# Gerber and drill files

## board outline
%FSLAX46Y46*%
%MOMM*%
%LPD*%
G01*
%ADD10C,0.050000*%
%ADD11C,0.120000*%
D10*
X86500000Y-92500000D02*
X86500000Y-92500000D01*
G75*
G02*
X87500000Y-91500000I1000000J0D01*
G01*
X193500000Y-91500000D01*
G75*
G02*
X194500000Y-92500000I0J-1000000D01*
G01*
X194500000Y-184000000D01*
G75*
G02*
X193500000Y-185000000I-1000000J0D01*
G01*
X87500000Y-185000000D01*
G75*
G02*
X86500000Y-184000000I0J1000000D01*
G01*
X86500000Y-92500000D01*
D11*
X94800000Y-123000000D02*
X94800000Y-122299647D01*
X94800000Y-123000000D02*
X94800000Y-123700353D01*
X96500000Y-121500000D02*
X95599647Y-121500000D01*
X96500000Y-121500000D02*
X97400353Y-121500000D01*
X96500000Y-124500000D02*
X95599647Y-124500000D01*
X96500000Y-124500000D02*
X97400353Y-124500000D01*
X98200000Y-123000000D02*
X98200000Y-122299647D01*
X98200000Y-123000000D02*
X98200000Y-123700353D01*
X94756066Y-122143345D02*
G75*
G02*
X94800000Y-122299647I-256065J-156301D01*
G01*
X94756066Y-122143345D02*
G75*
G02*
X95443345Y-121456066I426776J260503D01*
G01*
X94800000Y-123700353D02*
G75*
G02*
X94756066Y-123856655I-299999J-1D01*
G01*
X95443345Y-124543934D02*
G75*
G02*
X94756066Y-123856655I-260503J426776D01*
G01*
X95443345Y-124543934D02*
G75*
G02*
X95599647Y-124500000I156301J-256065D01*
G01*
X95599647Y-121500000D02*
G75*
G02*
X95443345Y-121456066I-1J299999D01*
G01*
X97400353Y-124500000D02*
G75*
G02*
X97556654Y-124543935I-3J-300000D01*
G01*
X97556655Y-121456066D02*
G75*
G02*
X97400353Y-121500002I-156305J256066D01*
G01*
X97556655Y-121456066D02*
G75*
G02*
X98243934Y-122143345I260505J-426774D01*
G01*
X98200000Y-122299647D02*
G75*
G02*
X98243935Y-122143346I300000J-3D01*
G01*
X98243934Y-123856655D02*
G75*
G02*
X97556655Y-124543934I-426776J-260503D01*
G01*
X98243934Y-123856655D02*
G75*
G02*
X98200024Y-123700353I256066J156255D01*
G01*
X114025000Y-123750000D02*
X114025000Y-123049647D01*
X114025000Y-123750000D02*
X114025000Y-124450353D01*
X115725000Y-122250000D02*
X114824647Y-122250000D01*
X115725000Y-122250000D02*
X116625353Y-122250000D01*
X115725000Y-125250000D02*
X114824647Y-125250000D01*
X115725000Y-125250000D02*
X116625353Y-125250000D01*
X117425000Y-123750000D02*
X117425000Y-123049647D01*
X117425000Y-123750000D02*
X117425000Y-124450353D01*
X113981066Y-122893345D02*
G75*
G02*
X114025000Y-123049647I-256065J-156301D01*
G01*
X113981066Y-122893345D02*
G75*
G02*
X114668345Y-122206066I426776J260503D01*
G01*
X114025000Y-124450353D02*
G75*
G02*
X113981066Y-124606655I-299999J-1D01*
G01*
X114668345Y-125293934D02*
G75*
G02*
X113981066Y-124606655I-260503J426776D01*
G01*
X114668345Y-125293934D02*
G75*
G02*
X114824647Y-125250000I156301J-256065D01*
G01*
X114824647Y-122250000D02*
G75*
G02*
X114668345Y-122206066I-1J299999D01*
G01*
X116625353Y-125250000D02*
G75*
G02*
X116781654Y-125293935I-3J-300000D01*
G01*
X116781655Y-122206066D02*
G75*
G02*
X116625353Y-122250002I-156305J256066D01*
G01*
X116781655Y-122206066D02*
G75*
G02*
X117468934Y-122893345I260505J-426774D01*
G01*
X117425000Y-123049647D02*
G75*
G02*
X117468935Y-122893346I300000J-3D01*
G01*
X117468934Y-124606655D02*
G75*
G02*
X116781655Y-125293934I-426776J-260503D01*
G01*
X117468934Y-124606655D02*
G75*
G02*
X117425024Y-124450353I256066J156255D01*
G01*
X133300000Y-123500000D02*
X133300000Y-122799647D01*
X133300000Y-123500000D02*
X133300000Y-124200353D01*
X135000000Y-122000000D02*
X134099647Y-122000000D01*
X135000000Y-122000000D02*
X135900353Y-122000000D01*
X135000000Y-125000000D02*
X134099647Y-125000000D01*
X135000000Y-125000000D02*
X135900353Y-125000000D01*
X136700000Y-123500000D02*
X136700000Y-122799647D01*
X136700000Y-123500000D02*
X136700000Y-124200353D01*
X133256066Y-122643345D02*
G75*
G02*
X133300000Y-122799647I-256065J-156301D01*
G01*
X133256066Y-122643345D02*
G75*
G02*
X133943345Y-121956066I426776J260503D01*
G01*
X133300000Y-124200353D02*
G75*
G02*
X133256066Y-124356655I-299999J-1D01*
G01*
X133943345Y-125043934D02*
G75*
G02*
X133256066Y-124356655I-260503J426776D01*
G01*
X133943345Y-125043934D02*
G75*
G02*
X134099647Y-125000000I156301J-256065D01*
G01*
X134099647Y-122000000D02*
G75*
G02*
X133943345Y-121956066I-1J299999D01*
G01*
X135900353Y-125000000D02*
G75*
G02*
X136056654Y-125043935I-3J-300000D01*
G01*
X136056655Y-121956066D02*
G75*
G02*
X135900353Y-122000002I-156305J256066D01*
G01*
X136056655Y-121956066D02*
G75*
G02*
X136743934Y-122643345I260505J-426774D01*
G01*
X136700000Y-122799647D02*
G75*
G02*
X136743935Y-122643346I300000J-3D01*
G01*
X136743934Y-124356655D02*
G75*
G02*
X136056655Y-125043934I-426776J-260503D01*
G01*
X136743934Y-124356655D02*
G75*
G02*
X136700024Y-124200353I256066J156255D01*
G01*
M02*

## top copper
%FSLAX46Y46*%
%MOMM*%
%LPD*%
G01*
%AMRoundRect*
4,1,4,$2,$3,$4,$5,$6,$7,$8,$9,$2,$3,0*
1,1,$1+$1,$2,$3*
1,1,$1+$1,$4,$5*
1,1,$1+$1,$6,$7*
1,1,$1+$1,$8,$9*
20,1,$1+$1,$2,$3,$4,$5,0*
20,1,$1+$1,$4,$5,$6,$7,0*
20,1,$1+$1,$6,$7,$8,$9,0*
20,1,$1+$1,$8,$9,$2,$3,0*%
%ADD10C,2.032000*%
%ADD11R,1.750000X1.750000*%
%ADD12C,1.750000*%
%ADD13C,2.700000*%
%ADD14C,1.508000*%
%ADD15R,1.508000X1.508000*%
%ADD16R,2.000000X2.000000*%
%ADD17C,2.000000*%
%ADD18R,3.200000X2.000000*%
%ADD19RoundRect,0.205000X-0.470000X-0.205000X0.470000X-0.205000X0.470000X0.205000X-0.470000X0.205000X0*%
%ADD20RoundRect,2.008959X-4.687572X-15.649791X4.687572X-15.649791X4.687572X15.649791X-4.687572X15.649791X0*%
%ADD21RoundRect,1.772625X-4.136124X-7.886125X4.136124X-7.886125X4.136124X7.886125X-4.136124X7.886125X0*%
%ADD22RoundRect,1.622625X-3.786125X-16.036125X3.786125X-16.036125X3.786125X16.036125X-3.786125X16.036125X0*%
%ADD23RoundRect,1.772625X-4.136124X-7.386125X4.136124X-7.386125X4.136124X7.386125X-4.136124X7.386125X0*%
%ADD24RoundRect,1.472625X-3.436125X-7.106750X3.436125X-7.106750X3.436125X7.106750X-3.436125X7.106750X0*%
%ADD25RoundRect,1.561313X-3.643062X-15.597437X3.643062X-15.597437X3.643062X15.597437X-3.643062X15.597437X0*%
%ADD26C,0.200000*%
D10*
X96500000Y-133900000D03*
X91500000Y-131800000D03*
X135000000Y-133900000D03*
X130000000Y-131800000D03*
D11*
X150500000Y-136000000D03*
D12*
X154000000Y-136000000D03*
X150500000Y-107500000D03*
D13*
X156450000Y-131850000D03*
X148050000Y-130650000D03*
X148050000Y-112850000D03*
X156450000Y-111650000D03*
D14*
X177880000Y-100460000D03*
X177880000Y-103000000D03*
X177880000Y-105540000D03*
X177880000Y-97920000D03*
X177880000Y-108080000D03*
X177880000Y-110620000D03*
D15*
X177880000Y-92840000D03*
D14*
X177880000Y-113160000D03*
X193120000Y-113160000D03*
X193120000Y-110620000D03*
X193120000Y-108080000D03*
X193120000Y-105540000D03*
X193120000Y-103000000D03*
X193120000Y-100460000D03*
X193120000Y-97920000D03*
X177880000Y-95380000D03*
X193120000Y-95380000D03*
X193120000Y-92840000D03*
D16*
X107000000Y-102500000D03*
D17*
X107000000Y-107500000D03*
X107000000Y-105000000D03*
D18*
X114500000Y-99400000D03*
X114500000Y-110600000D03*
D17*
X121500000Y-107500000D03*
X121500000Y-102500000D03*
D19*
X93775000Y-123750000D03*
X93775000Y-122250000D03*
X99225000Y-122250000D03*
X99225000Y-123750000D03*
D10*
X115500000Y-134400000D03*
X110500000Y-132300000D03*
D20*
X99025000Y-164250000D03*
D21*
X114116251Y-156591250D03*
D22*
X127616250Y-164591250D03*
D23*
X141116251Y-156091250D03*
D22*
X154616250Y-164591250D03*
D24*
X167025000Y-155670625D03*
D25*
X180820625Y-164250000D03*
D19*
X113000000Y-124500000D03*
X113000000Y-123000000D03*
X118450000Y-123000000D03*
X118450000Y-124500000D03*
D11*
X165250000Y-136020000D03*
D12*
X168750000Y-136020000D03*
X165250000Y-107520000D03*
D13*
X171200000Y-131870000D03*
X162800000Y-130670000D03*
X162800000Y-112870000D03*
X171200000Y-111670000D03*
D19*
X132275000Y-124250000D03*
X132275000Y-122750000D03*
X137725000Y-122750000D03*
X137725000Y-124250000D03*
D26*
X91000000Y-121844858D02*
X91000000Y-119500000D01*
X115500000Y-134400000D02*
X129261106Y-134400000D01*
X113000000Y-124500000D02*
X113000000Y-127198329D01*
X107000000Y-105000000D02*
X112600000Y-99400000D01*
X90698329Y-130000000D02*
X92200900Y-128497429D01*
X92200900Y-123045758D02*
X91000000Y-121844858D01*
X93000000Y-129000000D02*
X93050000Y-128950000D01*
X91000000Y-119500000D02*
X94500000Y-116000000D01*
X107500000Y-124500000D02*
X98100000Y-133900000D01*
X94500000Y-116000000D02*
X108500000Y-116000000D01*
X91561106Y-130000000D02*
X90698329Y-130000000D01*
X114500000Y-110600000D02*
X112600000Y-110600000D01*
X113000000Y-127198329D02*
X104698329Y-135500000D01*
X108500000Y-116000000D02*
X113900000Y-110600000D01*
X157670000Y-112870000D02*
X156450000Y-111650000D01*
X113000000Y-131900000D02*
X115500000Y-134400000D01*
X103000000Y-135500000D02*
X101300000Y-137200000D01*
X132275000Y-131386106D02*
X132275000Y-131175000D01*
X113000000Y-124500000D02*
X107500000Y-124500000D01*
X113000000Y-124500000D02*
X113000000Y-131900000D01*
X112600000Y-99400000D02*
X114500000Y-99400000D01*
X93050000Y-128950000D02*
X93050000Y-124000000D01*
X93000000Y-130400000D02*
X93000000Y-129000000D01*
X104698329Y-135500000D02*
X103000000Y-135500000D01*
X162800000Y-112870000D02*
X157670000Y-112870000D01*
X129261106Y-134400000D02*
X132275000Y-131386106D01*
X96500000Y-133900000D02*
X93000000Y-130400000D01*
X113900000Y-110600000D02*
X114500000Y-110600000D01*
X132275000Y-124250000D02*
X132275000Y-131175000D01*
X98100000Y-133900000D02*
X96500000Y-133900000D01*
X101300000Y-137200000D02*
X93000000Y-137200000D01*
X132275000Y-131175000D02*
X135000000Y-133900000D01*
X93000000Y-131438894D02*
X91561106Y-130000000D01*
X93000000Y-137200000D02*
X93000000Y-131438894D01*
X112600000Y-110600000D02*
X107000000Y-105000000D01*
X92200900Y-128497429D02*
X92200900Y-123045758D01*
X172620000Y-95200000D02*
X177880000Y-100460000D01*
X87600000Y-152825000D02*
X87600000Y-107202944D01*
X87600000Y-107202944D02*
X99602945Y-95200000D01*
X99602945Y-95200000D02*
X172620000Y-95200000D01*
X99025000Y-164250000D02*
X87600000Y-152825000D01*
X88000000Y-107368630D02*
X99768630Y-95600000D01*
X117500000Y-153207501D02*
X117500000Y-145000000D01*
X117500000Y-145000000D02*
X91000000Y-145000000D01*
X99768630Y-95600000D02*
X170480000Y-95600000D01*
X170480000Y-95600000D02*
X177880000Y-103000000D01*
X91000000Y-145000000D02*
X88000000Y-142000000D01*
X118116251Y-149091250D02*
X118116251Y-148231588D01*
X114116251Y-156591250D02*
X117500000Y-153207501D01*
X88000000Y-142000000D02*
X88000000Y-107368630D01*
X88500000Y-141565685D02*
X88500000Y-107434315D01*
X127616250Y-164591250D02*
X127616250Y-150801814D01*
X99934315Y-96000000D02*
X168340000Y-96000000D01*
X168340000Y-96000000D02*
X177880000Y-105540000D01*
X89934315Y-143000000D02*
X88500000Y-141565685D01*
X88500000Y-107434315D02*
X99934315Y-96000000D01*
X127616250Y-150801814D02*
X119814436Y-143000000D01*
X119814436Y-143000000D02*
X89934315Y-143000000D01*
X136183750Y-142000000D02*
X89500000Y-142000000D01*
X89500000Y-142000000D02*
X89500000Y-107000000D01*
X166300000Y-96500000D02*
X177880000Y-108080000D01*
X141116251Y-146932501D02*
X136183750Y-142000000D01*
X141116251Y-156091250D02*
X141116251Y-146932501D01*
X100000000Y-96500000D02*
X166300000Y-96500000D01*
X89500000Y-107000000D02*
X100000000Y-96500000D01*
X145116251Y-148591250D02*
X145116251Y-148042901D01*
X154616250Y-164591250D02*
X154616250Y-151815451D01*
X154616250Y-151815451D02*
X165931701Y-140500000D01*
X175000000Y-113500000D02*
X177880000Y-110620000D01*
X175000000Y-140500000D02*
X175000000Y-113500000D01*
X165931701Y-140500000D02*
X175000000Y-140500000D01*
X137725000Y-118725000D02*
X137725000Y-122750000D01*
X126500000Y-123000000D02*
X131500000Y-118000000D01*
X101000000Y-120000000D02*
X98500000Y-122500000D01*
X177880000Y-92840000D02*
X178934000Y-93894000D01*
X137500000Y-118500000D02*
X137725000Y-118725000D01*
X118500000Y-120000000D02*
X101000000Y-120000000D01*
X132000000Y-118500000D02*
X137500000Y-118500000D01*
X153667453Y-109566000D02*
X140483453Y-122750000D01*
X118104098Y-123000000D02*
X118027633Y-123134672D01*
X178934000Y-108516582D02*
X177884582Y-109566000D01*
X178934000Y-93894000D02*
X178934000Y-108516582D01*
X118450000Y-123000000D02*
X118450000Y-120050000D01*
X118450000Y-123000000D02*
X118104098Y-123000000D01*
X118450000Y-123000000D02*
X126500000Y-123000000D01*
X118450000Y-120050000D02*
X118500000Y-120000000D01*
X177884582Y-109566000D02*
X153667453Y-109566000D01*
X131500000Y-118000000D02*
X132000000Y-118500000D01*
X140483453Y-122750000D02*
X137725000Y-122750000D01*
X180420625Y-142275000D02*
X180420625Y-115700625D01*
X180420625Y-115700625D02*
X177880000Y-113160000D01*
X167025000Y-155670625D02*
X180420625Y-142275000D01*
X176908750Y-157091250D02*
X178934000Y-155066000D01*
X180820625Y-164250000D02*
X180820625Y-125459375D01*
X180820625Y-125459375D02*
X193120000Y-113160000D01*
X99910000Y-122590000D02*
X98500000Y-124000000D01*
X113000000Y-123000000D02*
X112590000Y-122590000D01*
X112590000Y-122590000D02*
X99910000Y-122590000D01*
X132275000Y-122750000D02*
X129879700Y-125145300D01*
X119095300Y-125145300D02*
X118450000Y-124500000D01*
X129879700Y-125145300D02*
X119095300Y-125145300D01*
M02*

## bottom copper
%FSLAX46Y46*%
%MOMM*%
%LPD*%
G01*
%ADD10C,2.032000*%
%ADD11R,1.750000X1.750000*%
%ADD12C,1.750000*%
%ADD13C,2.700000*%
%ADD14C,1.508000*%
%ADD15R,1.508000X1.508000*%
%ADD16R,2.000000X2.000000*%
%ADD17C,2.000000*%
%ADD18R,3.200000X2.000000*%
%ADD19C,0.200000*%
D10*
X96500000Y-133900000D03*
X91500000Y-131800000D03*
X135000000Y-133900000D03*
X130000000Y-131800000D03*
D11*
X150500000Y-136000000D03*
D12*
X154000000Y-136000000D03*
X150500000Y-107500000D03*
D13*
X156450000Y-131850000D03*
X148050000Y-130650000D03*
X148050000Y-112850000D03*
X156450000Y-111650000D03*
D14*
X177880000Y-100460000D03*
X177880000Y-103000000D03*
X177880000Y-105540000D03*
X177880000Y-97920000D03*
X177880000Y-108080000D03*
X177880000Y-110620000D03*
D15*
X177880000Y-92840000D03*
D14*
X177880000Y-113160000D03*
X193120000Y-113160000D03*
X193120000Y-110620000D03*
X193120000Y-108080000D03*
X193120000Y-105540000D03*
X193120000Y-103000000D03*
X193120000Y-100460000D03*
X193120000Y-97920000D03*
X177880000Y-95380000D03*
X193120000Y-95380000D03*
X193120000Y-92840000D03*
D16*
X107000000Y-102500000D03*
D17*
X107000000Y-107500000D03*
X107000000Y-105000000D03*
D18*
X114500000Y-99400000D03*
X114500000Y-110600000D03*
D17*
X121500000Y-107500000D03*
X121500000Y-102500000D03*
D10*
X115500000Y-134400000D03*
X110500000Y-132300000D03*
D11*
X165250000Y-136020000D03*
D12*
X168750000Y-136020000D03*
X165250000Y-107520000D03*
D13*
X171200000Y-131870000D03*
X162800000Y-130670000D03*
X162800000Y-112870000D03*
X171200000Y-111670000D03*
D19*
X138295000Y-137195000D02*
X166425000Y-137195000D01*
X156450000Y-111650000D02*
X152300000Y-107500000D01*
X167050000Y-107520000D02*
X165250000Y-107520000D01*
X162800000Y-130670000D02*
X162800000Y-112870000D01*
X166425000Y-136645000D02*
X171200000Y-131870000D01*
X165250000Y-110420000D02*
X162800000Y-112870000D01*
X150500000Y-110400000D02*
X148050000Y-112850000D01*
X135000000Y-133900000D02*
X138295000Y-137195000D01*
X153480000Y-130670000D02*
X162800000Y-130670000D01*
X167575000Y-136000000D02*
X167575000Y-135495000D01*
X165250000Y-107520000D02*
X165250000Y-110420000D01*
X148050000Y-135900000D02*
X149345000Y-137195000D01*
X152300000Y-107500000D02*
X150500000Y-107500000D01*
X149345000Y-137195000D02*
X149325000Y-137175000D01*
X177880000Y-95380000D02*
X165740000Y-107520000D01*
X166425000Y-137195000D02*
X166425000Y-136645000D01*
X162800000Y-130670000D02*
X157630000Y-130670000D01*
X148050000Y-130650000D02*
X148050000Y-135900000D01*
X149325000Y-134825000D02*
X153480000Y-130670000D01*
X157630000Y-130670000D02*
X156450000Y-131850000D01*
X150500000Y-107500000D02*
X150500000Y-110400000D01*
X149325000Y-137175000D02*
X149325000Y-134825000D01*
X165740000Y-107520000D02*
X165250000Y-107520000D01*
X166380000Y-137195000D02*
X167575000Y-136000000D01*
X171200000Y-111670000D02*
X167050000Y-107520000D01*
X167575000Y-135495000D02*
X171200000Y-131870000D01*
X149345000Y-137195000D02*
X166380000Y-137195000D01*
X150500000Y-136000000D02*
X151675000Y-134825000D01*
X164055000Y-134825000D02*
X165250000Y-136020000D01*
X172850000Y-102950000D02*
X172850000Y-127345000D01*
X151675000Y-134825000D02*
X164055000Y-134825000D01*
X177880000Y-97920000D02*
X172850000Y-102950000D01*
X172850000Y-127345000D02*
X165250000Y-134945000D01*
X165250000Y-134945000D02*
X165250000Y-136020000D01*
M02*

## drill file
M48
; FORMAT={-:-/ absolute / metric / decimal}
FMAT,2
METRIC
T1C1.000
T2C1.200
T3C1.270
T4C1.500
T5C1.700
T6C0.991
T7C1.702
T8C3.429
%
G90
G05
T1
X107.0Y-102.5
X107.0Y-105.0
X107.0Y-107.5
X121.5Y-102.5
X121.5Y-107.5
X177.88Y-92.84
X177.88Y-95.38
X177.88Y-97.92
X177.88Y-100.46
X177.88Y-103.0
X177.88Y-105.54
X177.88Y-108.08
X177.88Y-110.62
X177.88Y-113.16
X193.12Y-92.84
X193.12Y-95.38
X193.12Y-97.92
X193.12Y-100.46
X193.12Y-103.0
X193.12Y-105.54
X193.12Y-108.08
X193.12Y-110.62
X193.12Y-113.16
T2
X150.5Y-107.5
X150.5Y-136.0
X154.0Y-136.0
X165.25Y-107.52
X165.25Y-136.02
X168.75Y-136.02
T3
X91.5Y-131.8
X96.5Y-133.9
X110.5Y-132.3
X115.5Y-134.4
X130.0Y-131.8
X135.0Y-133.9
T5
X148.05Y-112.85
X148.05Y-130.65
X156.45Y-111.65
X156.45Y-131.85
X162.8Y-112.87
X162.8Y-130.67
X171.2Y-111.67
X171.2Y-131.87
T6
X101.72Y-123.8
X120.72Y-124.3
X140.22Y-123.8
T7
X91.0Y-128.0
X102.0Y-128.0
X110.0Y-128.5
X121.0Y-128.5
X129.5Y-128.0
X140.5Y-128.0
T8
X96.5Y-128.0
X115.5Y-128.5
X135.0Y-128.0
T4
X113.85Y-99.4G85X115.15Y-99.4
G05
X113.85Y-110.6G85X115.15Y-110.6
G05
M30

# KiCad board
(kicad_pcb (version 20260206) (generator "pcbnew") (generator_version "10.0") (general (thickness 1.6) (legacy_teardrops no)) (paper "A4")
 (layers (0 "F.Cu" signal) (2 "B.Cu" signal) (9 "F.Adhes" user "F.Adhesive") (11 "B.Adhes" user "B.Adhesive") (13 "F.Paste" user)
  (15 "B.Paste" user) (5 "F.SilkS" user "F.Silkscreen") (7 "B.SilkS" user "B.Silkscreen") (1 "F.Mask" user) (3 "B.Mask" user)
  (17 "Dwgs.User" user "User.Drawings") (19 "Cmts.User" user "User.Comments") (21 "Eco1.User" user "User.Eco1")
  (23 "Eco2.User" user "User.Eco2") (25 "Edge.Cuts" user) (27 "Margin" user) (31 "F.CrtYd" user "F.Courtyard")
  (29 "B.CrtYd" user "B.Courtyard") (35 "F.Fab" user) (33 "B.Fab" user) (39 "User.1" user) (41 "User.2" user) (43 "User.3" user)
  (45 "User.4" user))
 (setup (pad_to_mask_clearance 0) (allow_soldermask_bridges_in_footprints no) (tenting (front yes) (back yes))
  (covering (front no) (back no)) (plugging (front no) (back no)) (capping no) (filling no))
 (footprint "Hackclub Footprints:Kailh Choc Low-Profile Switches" (layer "F.Cu") (at 96.5 128)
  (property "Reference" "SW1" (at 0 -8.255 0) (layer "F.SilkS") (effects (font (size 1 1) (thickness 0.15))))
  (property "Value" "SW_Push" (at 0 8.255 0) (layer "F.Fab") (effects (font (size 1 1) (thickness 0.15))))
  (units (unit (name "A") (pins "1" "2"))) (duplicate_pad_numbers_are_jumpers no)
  (pad "" np_thru_hole circle (at -5.5 0) (size 1.7018 1.7018) (drill 1.7018) (layers "*.Cu" "*.Mask"))
  (pad "" np_thru_hole circle (at 0 0) (size 3.429 3.429) (drill 3.429) (layers "*.Cu" "*.Mask"))
  (pad "" np_thru_hole circle (at 5.22 -4.2) (size 0.9906 0.9906) (drill 0.9906) (layers "*.Cu" "*.Mask"))
  (pad "" np_thru_hole circle (at 5.5 0) (size 1.7018 1.7018) (drill 1.7018) (layers "*.Cu" "*.Mask"))
  (pad "1" thru_hole circle (at 0 5.9) (size 2.032 2.032) (drill 1.27) (layers "*.Cu" "*.Mask") (remove_unused_layers no) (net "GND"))
  (pad "2" thru_hole circle (at -5 3.8) (size 2.032 2.032) (drill 1.27) (layers "*.Cu" "*.Mask") (remove_unused_layers no) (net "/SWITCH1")))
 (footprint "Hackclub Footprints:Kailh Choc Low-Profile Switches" (layer "F.Cu") (at 135 128)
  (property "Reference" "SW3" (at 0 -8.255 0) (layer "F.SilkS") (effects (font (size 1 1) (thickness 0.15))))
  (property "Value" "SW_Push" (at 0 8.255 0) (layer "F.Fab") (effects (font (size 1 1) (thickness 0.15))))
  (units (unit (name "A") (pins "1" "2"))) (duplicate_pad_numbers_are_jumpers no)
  (pad "" np_thru_hole circle (at -5.5 0) (size 1.7018 1.7018) (drill 1.7018) (layers "*.Cu" "*.Mask"))
  (pad "" np_thru_hole circle (at 0 0) (size 3.429 3.429) (drill 3.429) (layers "*.Cu" "*.Mask"))
  (pad "" np_thru_hole circle (at 5.22 -4.2) (size 0.9906 0.9906) (drill 0.9906) (layers "*.Cu" "*.Mask"))
  (pad "" np_thru_hole circle (at 5.5 0) (size 1.7018 1.7018) (drill 1.7018) (layers "*.Cu" "*.Mask"))
  (pad "1" thru_hole circle (at 0 5.9) (size 2.032 2.032) (drill 1.27) (layers "*.Cu" "*.Mask") (remove_unused_layers no) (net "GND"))
  (pad "2" thru_hole circle (at -5 3.8) (size 2.032 2.032) (drill 1.27) (layers "*.Cu" "*.Mask") (remove_unused_layers no) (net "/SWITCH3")))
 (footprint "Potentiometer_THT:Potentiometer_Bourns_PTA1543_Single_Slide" (layer "F.Cu") (at 150.5 136 90)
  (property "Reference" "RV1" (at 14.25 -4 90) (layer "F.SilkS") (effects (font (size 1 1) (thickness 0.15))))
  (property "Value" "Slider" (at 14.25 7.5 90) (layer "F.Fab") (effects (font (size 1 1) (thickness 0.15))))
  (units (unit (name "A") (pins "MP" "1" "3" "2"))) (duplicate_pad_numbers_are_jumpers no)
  (pad "1" thru_hole rect (at 0 0 90) (size 1.75 1.75) (drill 1.2) (layers "*.Cu" "*.Mask") (remove_unused_layers no) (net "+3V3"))
  (pad "2" thru_hole circle (at 0 3.5 90) (size 1.75 1.75) (drill 1.2) (layers "*.Cu" "*.Mask") (remove_unused_layers no) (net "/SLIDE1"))
  (pad "3" thru_hole circle (at 28.5 0 90) (size 1.75 1.75) (drill 1.2) (layers "*.Cu" "*.Mask") (remove_unused_layers no) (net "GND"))
  (pad "MP" thru_hole circle (at 4.15 5.95 90) (size 2.7 2.7) (drill 1.7) (layers "*.Cu" "*.Mask") (remove_unused_layers no) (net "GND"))
  (pad "MP" thru_hole circle (at 5.35 -2.45 90) (size 2.7 2.7) (drill 1.7) (layers "*.Cu" "*.Mask") (remove_unused_layers no) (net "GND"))
  (pad "MP" thru_hole circle (at 23.15 -2.45 90) (size 2.7 2.7) (drill 1.7) (layers "*.Cu" "*.Mask") (remove_unused_layers no) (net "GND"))
  (pad "MP" thru_hole circle (at 24.35 5.95 90) (size 2.7 2.7) (drill 1.7) (layers "*.Cu" "*.Mask") (remove_unused_layers no) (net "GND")))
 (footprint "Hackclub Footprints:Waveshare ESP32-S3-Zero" (layer "F.Cu") (at 185.5 103)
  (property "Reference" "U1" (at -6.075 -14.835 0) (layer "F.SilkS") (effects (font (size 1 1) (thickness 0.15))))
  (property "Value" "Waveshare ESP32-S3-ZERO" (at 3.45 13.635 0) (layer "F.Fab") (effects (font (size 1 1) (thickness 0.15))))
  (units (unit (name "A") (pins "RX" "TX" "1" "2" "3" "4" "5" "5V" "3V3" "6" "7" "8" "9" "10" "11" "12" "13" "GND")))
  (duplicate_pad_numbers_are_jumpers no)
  (pad "1" thru_hole circle (at -7.62 -2.54) (size 1.508 1.508) (drill 1) (layers "*.Cu" "*.Mask") (remove_unused_layers no) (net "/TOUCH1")
   (solder_mask_margin 0.102))
  (pad "2" thru_hole circle (at -7.62 0) (size 1.508 1.508) (drill 1) (layers "*.Cu" "*.Mask") (remove_unused_layers no) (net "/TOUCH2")
   (solder_mask_margin 0.102))
  (pad "3" thru_hole circle (at -7.62 2.54) (size 1.508 1.508) (drill 1) (layers "*.Cu" "*.Mask") (remove_unused_layers no) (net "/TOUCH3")
   (solder_mask_margin 0.102))
  (pad "3V3" thru_hole circle (at -7.62 -5.08) (size 1.508 1.508) (drill 1) (layers "*.Cu" "*.Mask") (remove_unused_layers no) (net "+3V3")
   (solder_mask_margin 0.102))
  (pad "4" thru_hole circle (at -7.62 5.08) (size 1.508 1.508) (drill 1) (layers "*.Cu" "*.Mask") (remove_unused_layers no) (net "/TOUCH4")
   (solder_mask_margin 0.102))
  (pad "5" thru_hole circle (at -7.62 7.62) (size 1.508 1.508) (drill 1) (layers "*.Cu" "*.Mask") (remove_unused_layers no) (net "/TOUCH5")
   (solder_mask_margin 0.102))
  (pad "5V" thru_hole rect (at -7.62 -10.16) (size 1.508 1.508) (drill 1) (layers "*.Cu" "*.Mask") (remove_unused_layers no) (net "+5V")
   (solder_mask_margin 0.102))
  (pad "6" thru_hole circle (at -7.62 10.16) (size 1.508 1.508) (drill 1) (layers "*.Cu" "*.Mask") (remove_unused_layers no) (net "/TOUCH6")
   (solder_mask_margin 0.102))
  (pad "7" thru_hole circle (at 7.62 10.16) (size 1.508 1.508) (drill 1) (layers "*.Cu" "*.Mask") (remove_unused_layers no) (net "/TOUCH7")
   (solder_mask_margin 0.102))
  (pad "8" thru_hole circle (at 7.62 7.62) (size 1.508 1.508) (drill 1) (layers "*.Cu" "*.Mask") (remove_unused_layers no)
   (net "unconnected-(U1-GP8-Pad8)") (solder_mask_margin 0.102))
  (pad "9" thru_hole circle (at 7.62 5.08) (size 1.508 1.508) (drill 1) (layers "*.Cu" "*.Mask") (remove_unused_layers no)
   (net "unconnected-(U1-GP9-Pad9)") (solder_mask_margin 0.102))
  (pad "10" thru_hole circle (at 7.62 2.54) (size 1.508 1.508) (drill 1) (layers "*.Cu" "*.Mask") (remove_unused_layers no)
   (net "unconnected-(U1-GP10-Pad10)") (solder_mask_margin 0.102))
  (pad "11" thru_hole circle (at 7.62 0) (size 1.508 1.508) (drill 1) (layers "*.Cu" "*.Mask") (remove_unused_layers no)
   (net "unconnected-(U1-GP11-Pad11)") (solder_mask_margin 0.102))
  (pad "12" thru_hole circle (at 7.62 -2.54) (size 1.508 1.508) (drill 1) (layers "*.Cu" "*.Mask") (remove_unused_layers no)
   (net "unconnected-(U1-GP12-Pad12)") (solder_mask_margin 0.102))
  (pad "13" thru_hole circle (at 7.62 -5.08) (size 1.508 1.508) (drill 1) (layers "*.Cu" "*.Mask") (remove_unused_layers no)
   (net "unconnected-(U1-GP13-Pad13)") (solder_mask_margin 0.102))
  (pad "GND" thru_hole circle (at -7.62 -7.62) (size 1.508 1.508) (drill 1) (layers "*.Cu" "*.Mask") (remove_unused_layers no) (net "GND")
   (solder_mask_margin 0.102))
  (pad "RX" thru_hole circle (at 7.62 -7.62) (size 1.508 1.508) (drill 1) (layers "*.Cu" "*.Mask") (remove_unused_layers no)
   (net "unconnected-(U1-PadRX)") (solder_mask_margin 0.102))
  (pad "TX" thru_hole circle (at 7.62 -10.16) (size 1.508 1.508) (drill 1) (layers "*.Cu" "*.Mask") (remove_unused_layers no)
   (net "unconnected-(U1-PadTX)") (solder_mask_margin 0.102)))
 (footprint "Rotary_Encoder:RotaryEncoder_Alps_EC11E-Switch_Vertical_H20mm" (layer "F.Cu") (at 107 102.5)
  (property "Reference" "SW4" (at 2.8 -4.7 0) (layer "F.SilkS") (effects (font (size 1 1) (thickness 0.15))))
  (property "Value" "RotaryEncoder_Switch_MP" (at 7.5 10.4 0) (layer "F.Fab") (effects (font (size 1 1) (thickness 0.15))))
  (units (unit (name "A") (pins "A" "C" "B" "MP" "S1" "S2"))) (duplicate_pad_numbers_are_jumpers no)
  (pad "A" thru_hole rect (at 0 0) (size 2 2) (drill 1) (layers "*.Cu" "*.Mask") (remove_unused_layers no) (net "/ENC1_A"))
  (pad "B" thru_hole circle (at 0 5) (size 2 2) (drill 1) (layers "*.Cu" "*.Mask") (remove_unused_layers no) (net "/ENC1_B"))
  (pad "C" thru_hole circle (at 0 2.5) (size 2 2) (drill 1) (layers "*.Cu" "*.Mask") (remove_unused_layers no) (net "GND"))
  (pad "MP" thru_hole rect (at 7.5 -3.1) (size 3.2 2) (drill oval 2.8 1.5) (layers "*.Cu" "*.Mask") (remove_unused_layers no) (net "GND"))
  (pad "MP" thru_hole rect (at 7.5 8.1) (size 3.2 2) (drill oval 2.8 1.5) (layers "*.Cu" "*.Mask") (remove_unused_layers no) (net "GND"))
  (pad "S1" thru_hole circle (at 14.5 5) (size 2 2) (drill 1) (layers "*.Cu" "*.Mask") (remove_unused_layers no)
   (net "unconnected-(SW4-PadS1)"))
  (pad "S2" thru_hole circle (at 14.5 0) (size 2 2) (drill 1) (layers "*.Cu" "*.Mask") (remove_unused_layers no)
   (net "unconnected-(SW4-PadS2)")))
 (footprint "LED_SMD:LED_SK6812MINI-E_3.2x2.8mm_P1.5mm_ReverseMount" (layer "F.Cu") (at 96.5 123)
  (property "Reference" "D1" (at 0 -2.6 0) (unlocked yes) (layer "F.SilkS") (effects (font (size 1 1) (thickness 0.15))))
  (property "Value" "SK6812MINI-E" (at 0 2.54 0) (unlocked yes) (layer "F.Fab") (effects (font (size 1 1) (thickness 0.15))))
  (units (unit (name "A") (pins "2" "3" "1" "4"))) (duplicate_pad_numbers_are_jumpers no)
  (fp_line (start -1.7 0) (end -1.7 -0.700353) (stroke (width 0.12) (type solid)) (layer "Edge.Cuts"))
  (fp_line (start -1.7 0) (end -1.7 0.700353) (stroke (width 0.12) (type solid)) (layer "Edge.Cuts"))
  (fp_line (start 0 -1.5) (end -0.900353 -1.5) (stroke (width 0.12) (type solid)) (layer "Edge.Cuts"))
  (fp_line (start 0 -1.5) (end 0.900353 -1.5) (stroke (width 0.12) (type solid)) (layer "Edge.Cuts"))
  (fp_line (start 0 1.5) (end -0.900353 1.5) (stroke (width 0.12) (type solid)) (layer "Edge.Cuts"))
  (fp_line (start 0 1.5) (end 0.900353 1.5) (stroke (width 0.12) (type solid)) (layer "Edge.Cuts"))
  (fp_line (start 1.7 0) (end 1.7 -0.700353) (stroke (width 0.12) (type solid)) (layer "Edge.Cuts"))
  (fp_line (start 1.7 0) (end 1.7 0.700353) (stroke (width 0.12) (type solid)) (layer "Edge.Cuts"))
  (fp_arc (start -1.743934 -0.856655) (mid -1.711192 -0.781532) (end -1.7 -0.700353) (stroke (width 0.12) (type solid)) (layer "Edge.Cuts"))
  (fp_arc (start -1.743934 -0.856655) (mid -1.670711 -1.470711) (end -1.056655 -1.543934) (stroke (width 0.12) (type solid))
   (layer "Edge.Cuts"))
  (fp_arc (start -1.7 0.700353) (mid -1.711192 0.781532) (end -1.743934 0.856655) (stroke (width 0.12) (type solid)) (layer "Edge.Cuts"))
  (fp_arc (start -1.056655 1.543934) (mid -1.670711 1.470711) (end -1.743934 0.856655) (stroke (width 0.12) (type solid))
   (layer "Edge.Cuts"))
  (fp_arc (start -1.056655 1.543934) (mid -0.981532 1.511192) (end -0.900353 1.5) (stroke (width 0.12) (type solid)) (layer "Edge.Cuts"))
  (fp_arc (start -0.900353 -1.5) (mid -0.981532 -1.511192) (end -1.056655 -1.543934) (stroke (width 0.12) (type solid)) (layer "Edge.Cuts"))
  (fp_arc (start 0.900353 1.5) (mid 0.981532 1.511192) (end 1.056655 1.543934) (stroke (width 0.12) (type solid)) (layer "Edge.Cuts"))
  (fp_arc (start 1.056655 -1.543934) (mid 0.981532 -1.511192) (end 0.900353 -1.5) (stroke (width 0.12) (type solid)) (layer "Edge.Cuts"))
  (fp_arc (start 1.056655 -1.543934) (mid 1.670711 -1.470711) (end 1.743934 -0.856655) (stroke (width 0.12) (type solid))
   (layer "Edge.Cuts"))
  (fp_arc (start 1.7 -0.700353) (mid 1.711192 -0.781532) (end 1.743934 -0.856655) (stroke (width 0.12) (type solid)) (layer "Edge.Cuts"))
  (fp_arc (start 1.743934 0.856655) (mid 1.670711 1.470711) (end 1.056655 1.543934) (stroke (width 0.12) (type solid)) (layer "Edge.Cuts"))
  (fp_arc (start 1.743934 0.856655) (mid 1.711192 0.781532) (end 1.7 0.700353) (stroke (width 0.12) (type solid)) (layer "Edge.Cuts"))
  (pad "1" smd roundrect (at -2.725 0.75) (size 1.35 0.82) (layers "F.Cu" "F.Mask" "F.Paste") (roundrect_rratio 0.25) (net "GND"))
  (pad "2" smd roundrect (at -2.725 -0.75) (size 1.35 0.82) (layers "F.Cu" "F.Mask" "F.Paste") (roundrect_rratio 0.25) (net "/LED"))
  (pad "3" smd roundrect (at 2.725 -0.75) (size 1.35 0.82) (layers "F.Cu" "F.Mask" "F.Paste") (roundrect_rratio 0.25) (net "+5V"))
  (pad "4" smd roundrect (at 2.725 0.75) (size 1.35 0.82) (layers "F.Cu" "F.Mask" "F.Paste") (roundrect_rratio 0.25) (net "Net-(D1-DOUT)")))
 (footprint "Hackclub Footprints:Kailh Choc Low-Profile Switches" (layer "F.Cu") (at 115.5 128.5)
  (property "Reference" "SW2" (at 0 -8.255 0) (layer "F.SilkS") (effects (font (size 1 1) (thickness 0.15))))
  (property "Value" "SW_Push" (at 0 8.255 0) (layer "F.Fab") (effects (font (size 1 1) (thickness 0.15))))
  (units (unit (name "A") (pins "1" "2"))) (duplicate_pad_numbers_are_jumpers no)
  (pad "" np_thru_hole circle (at -5.5 0) (size 1.7018 1.7018) (drill 1.7018) (layers "*.Cu" "*.Mask"))
  (pad "" np_thru_hole circle (at 0 0) (size 3.429 3.429) (drill 3.429) (layers "*.Cu" "*.Mask"))
  (pad "" np_thru_hole circle (at 5.22 -4.2) (size 0.9906 0.9906) (drill 0.9906) (layers "*.Cu" "*.Mask"))
  (pad "" np_thru_hole circle (at 5.5 0) (size 1.7018 1.7018) (drill 1.7018) (layers "*.Cu" "*.Mask"))
  (pad "1" thru_hole circle (at 0 5.9) (size 2.032 2.032) (drill 1.27) (layers "*.Cu" "*.Mask") (remove_unused_layers no) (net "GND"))
  (pad "2" thru_hole circle (at -5 3.8) (size 2.032 2.032) (drill 1.27) (layers "*.Cu" "*.Mask") (remove_unused_layers no) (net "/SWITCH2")))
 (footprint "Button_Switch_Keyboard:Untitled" (layer "F.Cu") (at 141.025 142.25)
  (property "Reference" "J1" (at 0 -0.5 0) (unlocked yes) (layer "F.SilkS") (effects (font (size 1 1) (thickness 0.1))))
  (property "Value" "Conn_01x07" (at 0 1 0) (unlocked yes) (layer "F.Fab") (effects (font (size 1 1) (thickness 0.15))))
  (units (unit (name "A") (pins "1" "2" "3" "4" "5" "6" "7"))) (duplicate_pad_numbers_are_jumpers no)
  (pad "1" smd roundrect (at -42 22) (size 13.393062 35.3175) (layers "F.Cu" "F.Mask") (roundrect_rratio 0.15) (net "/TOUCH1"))
  (pad "2" smd roundrect (at -26.908749 14.34125) (size 11.817498 19.3175) (layers "F.Cu" "F.Mask") (roundrect_rratio 0.15) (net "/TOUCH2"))
  (pad "3" smd roundrect (at -13.40875 22.34125) (size 10.8175 35.3175) (layers "F.Cu" "F.Mask") (roundrect_rratio 0.15) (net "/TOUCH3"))
  (pad "4" smd roundrect (at 0.091251 13.84125) (size 11.817498 18.3175) (layers "F.Cu" "F.Mask") (roundrect_rratio 0.15) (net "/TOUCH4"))
  (pad "5" smd roundrect (at 13.59125 22.34125) (size 10.8175 35.3175) (layers "F.Cu" "F.Mask") (roundrect_rratio 0.15) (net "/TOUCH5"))
  (pad "6" smd roundrect (at 26 13.420625) (size 9.8175 17.15875) (layers "F.Cu" "F.Mask") (roundrect_rratio 0.15) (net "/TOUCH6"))
  (pad "7" smd roundrect (at 39.795625 22) (size 10.40875 34.3175) (layers "F.Cu" "F.Mask") (roundrect_rratio 0.15) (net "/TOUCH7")))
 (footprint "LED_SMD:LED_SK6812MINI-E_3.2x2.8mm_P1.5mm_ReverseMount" (layer "F.Cu") (at 115.725 123.75)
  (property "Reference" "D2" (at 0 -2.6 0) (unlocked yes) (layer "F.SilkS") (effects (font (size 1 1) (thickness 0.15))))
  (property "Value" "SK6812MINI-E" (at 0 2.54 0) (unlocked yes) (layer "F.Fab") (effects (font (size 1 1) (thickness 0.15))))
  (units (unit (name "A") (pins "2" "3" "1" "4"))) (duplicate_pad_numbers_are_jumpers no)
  (fp_line (start -1.7 0) (end -1.7 -0.700353) (stroke (width 0.12) (type solid)) (layer "Edge.Cuts"))
  (fp_line (start -1.7 0) (end -1.7 0.700353) (stroke (width 0.12) (type solid)) (layer "Edge.Cuts"))
  (fp_line (start 0 -1.5) (end -0.900353 -1.5) (stroke (width 0.12) (type solid)) (layer "Edge.Cuts"))
  (fp_line (start 0 -1.5) (end 0.900353 -1.5) (stroke (width 0.12) (type solid)) (layer "Edge.Cuts"))
  (fp_line (start 0 1.5) (end -0.900353 1.5) (stroke (width 0.12) (type solid)) (layer "Edge.Cuts"))
  (fp_line (start 0 1.5) (end 0.900353 1.5) (stroke (width 0.12) (type solid)) (layer "Edge.Cuts"))
  (fp_line (start 1.7 0) (end 1.7 -0.700353) (stroke (width 0.12) (type solid)) (layer "Edge.Cuts"))
  (fp_line (start 1.7 0) (end 1.7 0.700353) (stroke (width 0.12) (type solid)) (layer "Edge.Cuts"))
  (fp_arc (start -1.743934 -0.856655) (mid -1.711192 -0.781532) (end -1.7 -0.700353) (stroke (width 0.12) (type solid)) (layer "Edge.Cuts"))
  (fp_arc (start -1.743934 -0.856655) (mid -1.670711 -1.470711) (end -1.056655 -1.543934) (stroke (width 0.12) (type solid))
   (layer "Edge.Cuts"))
  (fp_arc (start -1.7 0.700353) (mid -1.711192 0.781532) (end -1.743934 0.856655) (stroke (width 0.12) (type solid)) (layer "Edge.Cuts"))
  (fp_arc (start -1.056655 1.543934) (mid -1.670711 1.470711) (end -1.743934 0.856655) (stroke (width 0.12) (type solid))
   (layer "Edge.Cuts"))
  (fp_arc (start -1.056655 1.543934) (mid -0.981532 1.511192) (end -0.900353 1.5) (stroke (width 0.12) (type solid)) (layer "Edge.Cuts"))
  (fp_arc (start -0.900353 -1.5) (mid -0.981532 -1.511192) (end -1.056655 -1.543934) (stroke (width 0.12) (type solid)) (layer "Edge.Cuts"))
  (fp_arc (start 0.900353 1.5) (mid 0.981532 1.511192) (end 1.056655 1.543934) (stroke (width 0.12) (type solid)) (layer "Edge.Cuts"))
  (fp_arc (start 1.056655 -1.543934) (mid 0.981532 -1.511192) (end 0.900353 -1.5) (stroke (width 0.12) (type solid)) (layer "Edge.Cuts"))
  (fp_arc (start 1.056655 -1.543934) (mid 1.670711 -1.470711) (end 1.743934 -0.856655) (stroke (width 0.12) (type solid))
   (layer "Edge.Cuts"))
  (fp_arc (start 1.7 -0.700353) (mid 1.711192 -0.781532) (end 1.743934 -0.856655) (stroke (width 0.12) (type solid)) (layer "Edge.Cuts"))
  (fp_arc (start 1.743934 0.856655) (mid 1.670711 1.470711) (end 1.056655 1.543934) (stroke (width 0.12) (type solid)) (layer "Edge.Cuts"))
  (fp_arc (start 1.743934 0.856655) (mid 1.711192 0.781532) (end 1.7 0.700353) (stroke (width 0.12) (type solid)) (layer "Edge.Cuts"))
  (pad "1" smd roundrect (at -2.725 0.75) (size 1.35 0.82) (layers "F.Cu" "F.Mask" "F.Paste") (roundrect_rratio 0.25) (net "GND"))
  (pad "2" smd roundrect (at -2.725 -0.75) (size 1.35 0.82) (layers "F.Cu" "F.Mask" "F.Paste") (roundrect_rratio 0.25) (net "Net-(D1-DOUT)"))
  (pad "3" smd roundrect (at 2.725 -0.75) (size 1.35 0.82) (layers "F.Cu" "F.Mask" "F.Paste") (roundrect_rratio 0.25) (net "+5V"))
  (pad "4" smd roundrect (at 2.725 0.75) (size 1.35 0.82) (layers "F.Cu" "F.Mask" "F.Paste") (roundrect_rratio 0.25) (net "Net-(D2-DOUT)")))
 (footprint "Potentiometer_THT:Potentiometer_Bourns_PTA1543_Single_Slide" (layer "F.Cu") (at 165.25 136.02 90)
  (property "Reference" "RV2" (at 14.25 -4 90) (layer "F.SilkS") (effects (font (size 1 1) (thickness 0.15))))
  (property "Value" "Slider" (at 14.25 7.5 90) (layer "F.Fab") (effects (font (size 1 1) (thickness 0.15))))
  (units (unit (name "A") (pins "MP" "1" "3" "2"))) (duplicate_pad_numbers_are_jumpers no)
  (pad "1" thru_hole rect (at 0 0 90) (size 1.75 1.75) (drill 1.2) (layers "*.Cu" "*.Mask") (remove_unused_layers no) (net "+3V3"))
  (pad "2" thru_hole circle (at 0 3.5 90) (size 1.75 1.75) (drill 1.2) (layers "*.Cu" "*.Mask") (remove_unused_layers no) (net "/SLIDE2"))
  (pad "3" thru_hole circle (at 28.5 0 90) (size 1.75 1.75) (drill 1.2) (layers "*.Cu" "*.Mask") (remove_unused_layers no) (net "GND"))
  (pad "MP" thru_hole circle (at 4.15 5.95 90) (size 2.7 2.7) (drill 1.7) (layers "*.Cu" "*.Mask") (remove_unused_layers no) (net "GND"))
  (pad "MP" thru_hole circle (at 5.35 -2.45 90) (size 2.7 2.7) (drill 1.7) (layers "*.Cu" "*.Mask") (remove_unused_layers no) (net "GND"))
  (pad "MP" thru_hole circle (at 23.15 -2.45 90) (size 2.7 2.7) (drill 1.7) (layers "*.Cu" "*.Mask") (remove_unused_layers no) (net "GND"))
  (pad "MP" thru_hole circle (at 24.35 5.95 90) (size 2.7 2.7) (drill 1.7) (layers "*.Cu" "*.Mask") (remove_unused_layers no) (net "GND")))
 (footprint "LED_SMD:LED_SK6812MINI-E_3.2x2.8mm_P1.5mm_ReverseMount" (layer "F.Cu") (at 135 123.5)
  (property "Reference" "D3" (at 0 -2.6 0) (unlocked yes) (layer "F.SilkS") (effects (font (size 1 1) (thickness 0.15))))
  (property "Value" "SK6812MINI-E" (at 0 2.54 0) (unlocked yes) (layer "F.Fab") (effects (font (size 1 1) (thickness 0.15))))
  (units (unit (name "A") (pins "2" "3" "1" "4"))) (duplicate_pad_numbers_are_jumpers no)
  (fp_line (start -1.7 0) (end -1.7 -0.700353) (stroke (width 0.12) (type solid)) (layer "Edge.Cuts"))
  (fp_line (start -1.7 0) (end -1.7 0.700353) (stroke (width 0.12) (type solid)) (layer "Edge.Cuts"))
  (fp_line (start 0 -1.5) (end -0.900353 -1.5) (stroke (width 0.12) (type solid)) (layer "Edge.Cuts"))
  (fp_line (start 0 -1.5) (end 0.900353 -1.5) (stroke (width 0.12) (type solid)) (layer "Edge.Cuts"))
  (fp_line (start 0 1.5) (end -0.900353 1.5) (stroke (width 0.12) (type solid)) (layer "Edge.Cuts"))
  (fp_line (start 0 1.5) (end 0.900353 1.5) (stroke (width 0.12) (type solid)) (layer "Edge.Cuts"))
  (fp_line (start 1.7 0) (end 1.7 -0.700353) (stroke (width 0.12) (type solid)) (layer "Edge.Cuts"))
  (fp_line (start 1.7 0) (end 1.7 0.700353) (stroke (width 0.12) (type solid)) (layer "Edge.Cuts"))
  (fp_arc (start -1.743934 -0.856655) (mid -1.711192 -0.781532) (end -1.7 -0.700353) (stroke (width 0.12) (type solid)) (layer "Edge.Cuts"))
  (fp_arc (start -1.743934 -0.856655) (mid -1.670711 -1.470711) (end -1.056655 -1.543934) (stroke (width 0.12) (type solid))
   (layer "Edge.Cuts"))
  (fp_arc (start -1.7 0.700353) (mid -1.711192 0.781532) (end -1.743934 0.856655) (stroke (width 0.12) (type solid)) (layer "Edge.Cuts"))
  (fp_arc (start -1.056655 1.543934) (mid -1.670711 1.470711) (end -1.743934 0.856655) (stroke (width 0.12) (type solid))
   (layer "Edge.Cuts"))
  (fp_arc (start -1.056655 1.543934) (mid -0.981532 1.511192) (end -0.900353 1.5) (stroke (width 0.12) (type solid)) (layer "Edge.Cuts"))
  (fp_arc (start -0.900353 -1.5) (mid -0.981532 -1.511192) (end -1.056655 -1.543934) (stroke (width 0.12) (type solid)) (layer "Edge.Cuts"))
  (fp_arc (start 0.900353 1.5) (mid 0.981532 1.511192) (end 1.056655 1.543934) (stroke (width 0.12) (type solid)) (layer "Edge.Cuts"))
  (fp_arc (start 1.056655 -1.543934) (mid 0.981532 -1.511192) (end 0.900353 -1.5) (stroke (width 0.12) (type solid)) (layer "Edge.Cuts"))
  (fp_arc (start 1.056655 -1.543934) (mid 1.670711 -1.470711) (end 1.743934 -0.856655) (stroke (width 0.12) (type solid))
   (layer "Edge.Cuts"))
  (fp_arc (start 1.7 -0.700353) (mid 1.711192 -0.781532) (end 1.743934 -0.856655) (stroke (width 0.12) (type solid)) (layer "Edge.Cuts"))
  (fp_arc (start 1.743934 0.856655) (mid 1.670711 1.470711) (end 1.056655 1.543934) (stroke (width 0.12) (type solid)) (layer "Edge.Cuts"))
  (fp_arc (start 1.743934 0.856655) (mid 1.711192 0.781532) (end 1.7 0.700353) (stroke (width 0.12) (type solid)) (layer "Edge.Cuts"))
  (pad "1" smd roundrect (at -2.725 0.75) (size 1.35 0.82) (layers "F.Cu" "F.Mask" "F.Paste") (roundrect_rratio 0.25) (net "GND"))
  (pad "2" smd roundrect (at -2.725 -0.75) (size 1.35 0.82) (layers "F.Cu" "F.Mask" "F.Paste") (roundrect_rratio 0.25) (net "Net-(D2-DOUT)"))
  (pad "3" smd roundrect (at 2.725 -0.75) (size 1.35 0.82) (layers "F.Cu" "F.Mask" "F.Paste") (roundrect_rratio 0.25) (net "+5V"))
  (pad "4" smd roundrect (at 2.725 0.75) (size 1.35 0.82) (layers "F.Cu" "F.Mask" "F.Paste") (roundrect_rratio 0.25)
   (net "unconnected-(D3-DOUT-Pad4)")))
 (gr_rect (start 86.5 91.5) (end 194.5 185) (radius 1) (stroke (width 0.05) (type solid)) (fill no) (layer "Edge.Cuts"))
 (segment (start 91 121.844858) (end 91 119.5) (width 0.2) (layer "F.Cu") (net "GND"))
 (segment (start 115.5 134.4) (end 129.261106 134.4) (width 0.2) (layer "F.Cu") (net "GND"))
 (segment (start 113 124.5) (end 113 127.198329) (width 0.2) (layer "F.Cu") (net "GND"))
 (segment (start 107 105) (end 112.6 99.4) (width 0.2) (layer "F.Cu") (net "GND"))
 (segment (start 90.698329 130) (end 92.2009 128.497429) (width 0.2) (layer "F.Cu") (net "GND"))
 (segment (start 92.2009 123.045758) (end 91 121.844858) (width 0.2) (layer "F.Cu") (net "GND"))
 (segment (start 93 129) (end 93.05 128.95) (width 0.2) (layer "F.Cu") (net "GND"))
 (segment (start 91 119.5) (end 94.5 116) (width 0.2) (layer "F.Cu") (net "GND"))
 (segment (start 107.5 124.5) (end 98.1 133.9) (width 0.2) (layer "F.Cu") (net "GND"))
 (segment (start 94.5 116) (end 108.5 116) (width 0.2) (layer "F.Cu") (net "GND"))
 (segment (start 91.561106 130) (end 90.698329 130) (width 0.2) (layer "F.Cu") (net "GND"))
 (segment (start 114.5 110.6) (end 112.6 110.6) (width 0.2) (layer "F.Cu") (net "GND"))
 (segment (start 113 127.198329) (end 104.698329 135.5) (width 0.2) (layer "F.Cu") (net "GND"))
 (segment (start 108.5 116) (end 113.9 110.6) (width 0.2) (layer "F.Cu") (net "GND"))
 (segment (start 157.67 112.87) (end 156.45 111.65) (width 0.2) (layer "F.Cu") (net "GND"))
 (segment (start 113 131.9) (end 115.5 134.4) (width 0.2) (layer "F.Cu") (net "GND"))
 (segment (start 103 135.5) (end 101.3 137.2) (width 0.2) (layer "F.Cu") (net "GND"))
 (segment (start 132.275 131.386106) (end 132.275 131.175) (width 0.2) (layer "F.Cu") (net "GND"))
 (segment (start 113 124.5) (end 107.5 124.5) (width 0.2) (layer "F.Cu") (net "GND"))
 (segment (start 113 124.5) (end 113 131.9) (width 0.2) (layer "F.Cu") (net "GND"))
 (segment (start 112.6 99.4) (end 114.5 99.4) (width 0.2) (layer "F.Cu") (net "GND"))
 (segment (start 93.05 128.95) (end 93.05 124) (width 0.2) (layer "F.Cu") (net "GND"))
 (segment (start 93 130.4) (end 93 129) (width 0.2) (layer "F.Cu") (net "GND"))
 (segment (start 104.698329 135.5) (end 103 135.5) (width 0.2) (layer "F.Cu") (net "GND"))
 (segment (start 162.8 112.87) (end 157.67 112.87) (width 0.2) (layer "F.Cu") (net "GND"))
 (segment (start 129.261106 134.4) (end 132.275 131.386106) (width 0.2) (layer "F.Cu") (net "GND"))
 (segment (start 96.5 133.9) (end 93 130.4) (width 0.2) (layer "F.Cu") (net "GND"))
 (segment (start 113.9 110.6) (end 114.5 110.6) (width 0.2) (layer "F.Cu") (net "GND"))
 (segment (start 132.275 124.25) (end 132.275 131.175) (width 0.2) (layer "F.Cu") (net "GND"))
 (segment (start 98.1 133.9) (end 96.5 133.9) (width 0.2) (layer "F.Cu") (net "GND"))
 (segment (start 101.3 137.2) (end 93 137.2) (width 0.2) (layer "F.Cu") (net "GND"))
 (segment (start 132.275 131.175) (end 135 133.9) (width 0.2) (layer "F.Cu") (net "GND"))
 (segment (start 93 131.438894) (end 91.561106 130) (width 0.2) (layer "F.Cu") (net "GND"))
 (segment (start 93 137.2) (end 93 131.438894) (width 0.2) (layer "F.Cu") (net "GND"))
 (segment (start 112.6 110.6) (end 107 105) (width 0.2) (layer "F.Cu") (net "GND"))
 (segment (start 92.2009 128.497429) (end 92.2009 123.045758) (width 0.2) (layer "F.Cu") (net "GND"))
 (segment (start 138.295 137.195) (end 166.425 137.195) (width 0.2) (layer "B.Cu") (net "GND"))
 (segment (start 156.45 111.65) (end 152.3 107.5) (width 0.2) (layer "B.Cu") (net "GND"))
 (segment (start 167.05 107.52) (end 165.25 107.52) (width 0.2) (layer "B.Cu") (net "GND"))
 (segment (start 162.8 130.67) (end 162.8 112.87) (width 0.2) (layer "B.Cu") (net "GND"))
 (segment (start 166.425 136.645) (end 171.2 131.87) (width 0.2) (layer "B.Cu") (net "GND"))
 (segment (start 165.25 110.42) (end 162.8 112.87) (width 0.2) (layer "B.Cu") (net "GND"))
 (segment (start 150.5 110.4) (end 148.05 112.85) (width 0.2) (layer "B.Cu") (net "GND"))
 (segment (start 135 133.9) (end 138.295 137.195) (width 0.2) (layer "B.Cu") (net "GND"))
 (segment (start 153.48 130.67) (end 162.8 130.67) (width 0.2) (layer "B.Cu") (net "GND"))
 (segment (start 167.575 136) (end 167.575 135.495) (width 0.2) (layer "B.Cu") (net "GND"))
 (segment (start 165.25 107.52) (end 165.25 110.42) (width 0.2) (layer "B.Cu") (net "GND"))
 (segment (start 148.05 135.9) (end 149.345 137.195) (width 0.2) (layer "B.Cu") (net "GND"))
 (segment (start 152.3 107.5) (end 150.5 107.5) (width 0.2) (layer "B.Cu") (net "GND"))
 (segment (start 149.345 137.195) (end 149.325 137.175) (width 0.2) (layer "B.Cu") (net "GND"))
 (segment (start 177.88 95.38) (end 165.74 107.52) (width 0.2) (layer "B.Cu") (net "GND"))
 (segment (start 166.425 137.195) (end 166.425 136.645) (width 0.2) (layer "B.Cu") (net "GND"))
 (segment (start 162.8 130.67) (end 157.63 130.67) (width 0.2) (layer "B.Cu") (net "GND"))
 (segment (start 148.05 130.65) (end 148.05 135.9) (width 0.2) (layer "B.Cu") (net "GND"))
 (segment (start 149.325 134.825) (end 153.48 130.67) (width 0.2) (layer "B.Cu") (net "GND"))
 (segment (start 157.63 130.67) (end 156.45 131.85) (width 0.2) (layer "B.Cu") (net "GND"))
 (segment (start 150.5 107.5) (end 150.5 110.4) (width 0.2) (layer "B.Cu") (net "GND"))
 (segment (start 149.325 137.175) (end 149.325 134.825) (width 0.2) (layer "B.Cu") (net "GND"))
 (segment (start 165.74 107.52) (end 165.25 107.52) (width 0.2) (layer "B.Cu") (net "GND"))
 (segment (start 166.38 137.195) (end 167.575 136) (width 0.2) (layer "B.Cu") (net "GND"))
 (segment (start 171.2 111.67) (end 167.05 107.52) (width 0.2) (layer "B.Cu") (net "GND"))
 (segment (start 167.575 135.495) (end 171.2 131.87) (width 0.2) (layer "B.Cu") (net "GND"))
 (segment (start 149.345 137.195) (end 166.38 137.195) (width 0.2) (layer "B.Cu") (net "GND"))
 (segment (start 150.5 136) (end 151.675 134.825) (width 0.2) (layer "B.Cu") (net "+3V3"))
 (segment (start 164.055 134.825) (end 165.25 136.02) (width 0.2) (layer "B.Cu") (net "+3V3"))
 (segment (start 172.85 102.95) (end 172.85 127.345) (width 0.2) (layer "B.Cu") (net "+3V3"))
 (segment (start 151.675 134.825) (end 164.055 134.825) (width 0.2) (layer "B.Cu") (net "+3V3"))
 (segment (start 177.88 97.92) (end 172.85 102.95) (width 0.2) (layer "B.Cu") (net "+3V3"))
 (segment (start 172.85 127.345) (end 165.25 134.945) (width 0.2) (layer "B.Cu") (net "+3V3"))
 (segment (start 165.25 134.945) (end 165.25 136.02) (width 0.2) (layer "B.Cu") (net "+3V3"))
 (segment (start 172.62 95.2) (end 177.88 100.46) (width 0.2) (layer "F.Cu") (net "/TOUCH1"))
 (segment (start 87.6 152.825) (end 87.6 107.202944) (width 0.2) (layer "F.Cu") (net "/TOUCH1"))
 (segment (start 87.6 107.202944) (end 99.602945 95.2) (width 0.2) (layer "F.Cu") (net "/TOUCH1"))
 (segment (start 99.602945 95.2) (end 172.62 95.2) (width 0.2) (layer "F.Cu") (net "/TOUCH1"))
 (segment (start 99.025 164.25) (end 87.6 152.825) (width 0.2) (layer "F.Cu") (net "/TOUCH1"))
 (segment (start 88 107.36863) (end 99.76863 95.6) (width 0.2) (layer "F.Cu") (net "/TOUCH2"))
 (segment (start 117.5 153.207501) (end 117.5 145) (width 0.2) (layer "F.Cu") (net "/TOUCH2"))
 (segment (start 117.5 145) (end 91 145) (width 0.2) (layer "F.Cu") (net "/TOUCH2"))
 (segment (start 99.76863 95.6) (end 170.48 95.6) (width 0.2) (layer "F.Cu") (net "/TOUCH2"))
 (segment (start 170.48 95.6) (end 177.88 103) (width 0.2) (layer "F.Cu") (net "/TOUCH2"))
 (segment (start 91 145) (end 88 142) (width 0.2) (layer "F.Cu") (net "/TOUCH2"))
 (segment (start 118.116251 149.09125) (end 118.116251 148.231588) (width 0.2) (layer "F.Cu") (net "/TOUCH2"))
 (segment (start 114.116251 156.59125) (end 117.5 153.207501) (width 0.2) (layer "F.Cu") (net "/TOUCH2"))
 (segment (start 88 142) (end 88 107.36863) (width 0.2) (layer "F.Cu") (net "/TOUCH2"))
 (segment (start 88.5 141.565685) (end 88.5 107.434315) (width 0.2) (layer "F.Cu") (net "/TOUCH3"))
 (segment (start 127.61625 164.59125) (end 127.61625 150.801814) (width 0.2) (layer "F.Cu") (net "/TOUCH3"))
 (segment (start 99.934315 96) (end 168.34 96) (width 0.2) (layer "F.Cu") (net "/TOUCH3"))
 (segment (start 168.34 96) (end 177.88 105.54) (width 0.2) (layer "F.Cu") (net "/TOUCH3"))
 (segment (start 89.934315 143) (end 88.5 141.565685) (width 0.2) (layer "F.Cu") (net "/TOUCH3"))
 (segment (start 88.5 107.434315) (end 99.934315 96) (width 0.2) (layer "F.Cu") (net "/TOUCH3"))
 (segment (start 127.61625 150.801814) (end 119.814436 143) (width 0.2) (layer "F.Cu") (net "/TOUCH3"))
 (segment (start 119.814436 143) (end 89.934315 143) (width 0.2) (layer "F.Cu") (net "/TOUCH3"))
 (segment (start 136.18375 142) (end 89.5 142) (width 0.2) (layer "F.Cu") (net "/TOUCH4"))
 (segment (start 89.5 142) (end 89.5 107) (width 0.2) (layer "F.Cu") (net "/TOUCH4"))
 (segment (start 166.3 96.5) (end 177.88 108.08) (width 0.2) (layer "F.Cu") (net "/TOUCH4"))
 (segment (start 141.116251 146.932501) (end 136.18375 142) (width 0.2) (layer "F.Cu") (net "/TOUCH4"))
 (segment (start 141.116251 156.09125) (end 141.116251 146.932501) (width 0.2) (layer "F.Cu") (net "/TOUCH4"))
 (segment (start 100 96.5) (end 166.3 96.5) (width 0.2) (layer "F.Cu") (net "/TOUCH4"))
 (segment (start 89.5 107) (end 100 96.5) (width 0.2) (layer "F.Cu") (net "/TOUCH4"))
 (segment (start 145.116251 148.59125) (end 145.116251 148.042901) (width 0.2) (layer "F.Cu") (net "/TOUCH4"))
 (segment (start 154.61625 164.59125) (end 154.61625 151.815451) (width 0.2) (layer "F.Cu") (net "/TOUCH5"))
 (segment (start 154.61625 151.815451) (end 165.931701 140.5) (width 0.2) (layer "F.Cu") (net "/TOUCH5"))
 (segment (start 175 113.5) (end 177.88 110.62) (width 0.2) (layer "F.Cu") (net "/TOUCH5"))
 (segment (start 175 140.5) (end 175 113.5) (width 0.2) (layer "F.Cu") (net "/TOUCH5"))
 (segment (start 165.931701 140.5) (end 175 140.5) (width 0.2) (layer "F.Cu") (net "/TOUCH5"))
 (segment (start 137.725 118.725) (end 137.725 122.75) (width 0.2) (layer "F.Cu") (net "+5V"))
 (segment (start 126.5 123) (end 131.5 118) (width 0.2) (layer "F.Cu") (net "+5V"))
 (segment (start 101 120) (end 98.5 122.5) (width 0.2) (layer "F.Cu") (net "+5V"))
 (segment (start 177.88 92.84) (end 178.934 93.894) (width 0.2) (layer "F.Cu") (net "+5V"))
 (segment (start 137.5 118.5) (end 137.725 118.725) (width 0.2) (layer "F.Cu") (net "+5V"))
 (segment (start 118.5 120) (end 101 120) (width 0.2) (layer "F.Cu") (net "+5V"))
 (segment (start 132 118.5) (end 137.5 118.5) (width 0.2) (layer "F.Cu") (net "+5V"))
 (segment (start 153.667453 109.566) (end 140.483453 122.75) (width 0.2) (layer "F.Cu") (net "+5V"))
 (segment (start 118.104098 123) (end 118.027633 123.134672) (width 0.2) (layer "F.Cu") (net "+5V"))
 (segment (start 178.934 108.516582) (end 177.884582 109.566) (width 0.2) (layer "F.Cu") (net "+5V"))
 (segment (start 178.934 93.894) (end 178.934 108.516582) (width 0.2) (layer "F.Cu") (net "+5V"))
 (segment (start 118.45 123) (end 118.45 120.05) (width 0.2) (layer "F.Cu") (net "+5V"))
 (segment (start 118.45 123) (end 118.104098 123) (width 0.2) (layer "F.Cu") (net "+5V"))
 (segment (start 118.45 123) (end 126.5 123) (width 0.2) (layer "F.Cu") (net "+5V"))
 (segment (start 118.45 120.05) (end 118.5 120) (width 0.2) (layer "F.Cu") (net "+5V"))
 (segment (start 177.884582 109.566) (end 153.667453 109.566) (width 0.2) (layer "F.Cu") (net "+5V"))
 (segment (start 131.5 118) (end 132 118.5) (width 0.2) (layer "F.Cu") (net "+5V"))
 (segment (start 140.483453 122.75) (end 137.725 122.75) (width 0.2) (layer "F.Cu") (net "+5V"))
 (segment (start 180.420625 142.275) (end 180.420625 115.700625) (width 0.2) (layer "F.Cu") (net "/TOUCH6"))
 (segment (start 180.420625 115.700625) (end 177.88 113.16) (width 0.2) (layer "F.Cu") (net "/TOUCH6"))
 (segment (start 167.025 155.670625) (end 180.420625 142.275) (width 0.2) (layer "F.Cu") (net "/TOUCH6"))
 (segment (start 176.90875 157.09125) (end 178.934 155.066) (width 0.2) (layer "F.Cu") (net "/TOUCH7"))
 (segment (start 180.820625 164.25) (end 180.820625 125.459375) (width 0.2) (layer "F.Cu") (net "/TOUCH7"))
 (segment (start 180.820625 125.459375) (end 193.12 113.16) (width 0.2) (layer "F.Cu") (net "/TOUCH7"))
 (segment (start 99.91 122.59) (end 98.5 124) (width 0.2) (layer "F.Cu") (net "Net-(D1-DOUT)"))
 (segment (start 113 123) (end 112.59 122.59) (width 0.2) (layer "F.Cu") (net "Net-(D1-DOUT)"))
 (segment (start 112.59 122.59) (end 99.91 122.59) (width 0.2) (layer "F.Cu") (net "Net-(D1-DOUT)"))
 (segment (start 132.275 122.75) (end 129.8797 125.1453) (width 0.2) (layer "F.Cu") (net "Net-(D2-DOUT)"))
 (segment (start 119.0953 125.1453) (end 118.45 124.5) (width 0.2) (layer "F.Cu") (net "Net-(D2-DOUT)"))
 (segment (start 129.8797 125.1453) (end 119.0953 125.1453) (width 0.2) (layer "F.Cu") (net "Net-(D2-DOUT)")))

